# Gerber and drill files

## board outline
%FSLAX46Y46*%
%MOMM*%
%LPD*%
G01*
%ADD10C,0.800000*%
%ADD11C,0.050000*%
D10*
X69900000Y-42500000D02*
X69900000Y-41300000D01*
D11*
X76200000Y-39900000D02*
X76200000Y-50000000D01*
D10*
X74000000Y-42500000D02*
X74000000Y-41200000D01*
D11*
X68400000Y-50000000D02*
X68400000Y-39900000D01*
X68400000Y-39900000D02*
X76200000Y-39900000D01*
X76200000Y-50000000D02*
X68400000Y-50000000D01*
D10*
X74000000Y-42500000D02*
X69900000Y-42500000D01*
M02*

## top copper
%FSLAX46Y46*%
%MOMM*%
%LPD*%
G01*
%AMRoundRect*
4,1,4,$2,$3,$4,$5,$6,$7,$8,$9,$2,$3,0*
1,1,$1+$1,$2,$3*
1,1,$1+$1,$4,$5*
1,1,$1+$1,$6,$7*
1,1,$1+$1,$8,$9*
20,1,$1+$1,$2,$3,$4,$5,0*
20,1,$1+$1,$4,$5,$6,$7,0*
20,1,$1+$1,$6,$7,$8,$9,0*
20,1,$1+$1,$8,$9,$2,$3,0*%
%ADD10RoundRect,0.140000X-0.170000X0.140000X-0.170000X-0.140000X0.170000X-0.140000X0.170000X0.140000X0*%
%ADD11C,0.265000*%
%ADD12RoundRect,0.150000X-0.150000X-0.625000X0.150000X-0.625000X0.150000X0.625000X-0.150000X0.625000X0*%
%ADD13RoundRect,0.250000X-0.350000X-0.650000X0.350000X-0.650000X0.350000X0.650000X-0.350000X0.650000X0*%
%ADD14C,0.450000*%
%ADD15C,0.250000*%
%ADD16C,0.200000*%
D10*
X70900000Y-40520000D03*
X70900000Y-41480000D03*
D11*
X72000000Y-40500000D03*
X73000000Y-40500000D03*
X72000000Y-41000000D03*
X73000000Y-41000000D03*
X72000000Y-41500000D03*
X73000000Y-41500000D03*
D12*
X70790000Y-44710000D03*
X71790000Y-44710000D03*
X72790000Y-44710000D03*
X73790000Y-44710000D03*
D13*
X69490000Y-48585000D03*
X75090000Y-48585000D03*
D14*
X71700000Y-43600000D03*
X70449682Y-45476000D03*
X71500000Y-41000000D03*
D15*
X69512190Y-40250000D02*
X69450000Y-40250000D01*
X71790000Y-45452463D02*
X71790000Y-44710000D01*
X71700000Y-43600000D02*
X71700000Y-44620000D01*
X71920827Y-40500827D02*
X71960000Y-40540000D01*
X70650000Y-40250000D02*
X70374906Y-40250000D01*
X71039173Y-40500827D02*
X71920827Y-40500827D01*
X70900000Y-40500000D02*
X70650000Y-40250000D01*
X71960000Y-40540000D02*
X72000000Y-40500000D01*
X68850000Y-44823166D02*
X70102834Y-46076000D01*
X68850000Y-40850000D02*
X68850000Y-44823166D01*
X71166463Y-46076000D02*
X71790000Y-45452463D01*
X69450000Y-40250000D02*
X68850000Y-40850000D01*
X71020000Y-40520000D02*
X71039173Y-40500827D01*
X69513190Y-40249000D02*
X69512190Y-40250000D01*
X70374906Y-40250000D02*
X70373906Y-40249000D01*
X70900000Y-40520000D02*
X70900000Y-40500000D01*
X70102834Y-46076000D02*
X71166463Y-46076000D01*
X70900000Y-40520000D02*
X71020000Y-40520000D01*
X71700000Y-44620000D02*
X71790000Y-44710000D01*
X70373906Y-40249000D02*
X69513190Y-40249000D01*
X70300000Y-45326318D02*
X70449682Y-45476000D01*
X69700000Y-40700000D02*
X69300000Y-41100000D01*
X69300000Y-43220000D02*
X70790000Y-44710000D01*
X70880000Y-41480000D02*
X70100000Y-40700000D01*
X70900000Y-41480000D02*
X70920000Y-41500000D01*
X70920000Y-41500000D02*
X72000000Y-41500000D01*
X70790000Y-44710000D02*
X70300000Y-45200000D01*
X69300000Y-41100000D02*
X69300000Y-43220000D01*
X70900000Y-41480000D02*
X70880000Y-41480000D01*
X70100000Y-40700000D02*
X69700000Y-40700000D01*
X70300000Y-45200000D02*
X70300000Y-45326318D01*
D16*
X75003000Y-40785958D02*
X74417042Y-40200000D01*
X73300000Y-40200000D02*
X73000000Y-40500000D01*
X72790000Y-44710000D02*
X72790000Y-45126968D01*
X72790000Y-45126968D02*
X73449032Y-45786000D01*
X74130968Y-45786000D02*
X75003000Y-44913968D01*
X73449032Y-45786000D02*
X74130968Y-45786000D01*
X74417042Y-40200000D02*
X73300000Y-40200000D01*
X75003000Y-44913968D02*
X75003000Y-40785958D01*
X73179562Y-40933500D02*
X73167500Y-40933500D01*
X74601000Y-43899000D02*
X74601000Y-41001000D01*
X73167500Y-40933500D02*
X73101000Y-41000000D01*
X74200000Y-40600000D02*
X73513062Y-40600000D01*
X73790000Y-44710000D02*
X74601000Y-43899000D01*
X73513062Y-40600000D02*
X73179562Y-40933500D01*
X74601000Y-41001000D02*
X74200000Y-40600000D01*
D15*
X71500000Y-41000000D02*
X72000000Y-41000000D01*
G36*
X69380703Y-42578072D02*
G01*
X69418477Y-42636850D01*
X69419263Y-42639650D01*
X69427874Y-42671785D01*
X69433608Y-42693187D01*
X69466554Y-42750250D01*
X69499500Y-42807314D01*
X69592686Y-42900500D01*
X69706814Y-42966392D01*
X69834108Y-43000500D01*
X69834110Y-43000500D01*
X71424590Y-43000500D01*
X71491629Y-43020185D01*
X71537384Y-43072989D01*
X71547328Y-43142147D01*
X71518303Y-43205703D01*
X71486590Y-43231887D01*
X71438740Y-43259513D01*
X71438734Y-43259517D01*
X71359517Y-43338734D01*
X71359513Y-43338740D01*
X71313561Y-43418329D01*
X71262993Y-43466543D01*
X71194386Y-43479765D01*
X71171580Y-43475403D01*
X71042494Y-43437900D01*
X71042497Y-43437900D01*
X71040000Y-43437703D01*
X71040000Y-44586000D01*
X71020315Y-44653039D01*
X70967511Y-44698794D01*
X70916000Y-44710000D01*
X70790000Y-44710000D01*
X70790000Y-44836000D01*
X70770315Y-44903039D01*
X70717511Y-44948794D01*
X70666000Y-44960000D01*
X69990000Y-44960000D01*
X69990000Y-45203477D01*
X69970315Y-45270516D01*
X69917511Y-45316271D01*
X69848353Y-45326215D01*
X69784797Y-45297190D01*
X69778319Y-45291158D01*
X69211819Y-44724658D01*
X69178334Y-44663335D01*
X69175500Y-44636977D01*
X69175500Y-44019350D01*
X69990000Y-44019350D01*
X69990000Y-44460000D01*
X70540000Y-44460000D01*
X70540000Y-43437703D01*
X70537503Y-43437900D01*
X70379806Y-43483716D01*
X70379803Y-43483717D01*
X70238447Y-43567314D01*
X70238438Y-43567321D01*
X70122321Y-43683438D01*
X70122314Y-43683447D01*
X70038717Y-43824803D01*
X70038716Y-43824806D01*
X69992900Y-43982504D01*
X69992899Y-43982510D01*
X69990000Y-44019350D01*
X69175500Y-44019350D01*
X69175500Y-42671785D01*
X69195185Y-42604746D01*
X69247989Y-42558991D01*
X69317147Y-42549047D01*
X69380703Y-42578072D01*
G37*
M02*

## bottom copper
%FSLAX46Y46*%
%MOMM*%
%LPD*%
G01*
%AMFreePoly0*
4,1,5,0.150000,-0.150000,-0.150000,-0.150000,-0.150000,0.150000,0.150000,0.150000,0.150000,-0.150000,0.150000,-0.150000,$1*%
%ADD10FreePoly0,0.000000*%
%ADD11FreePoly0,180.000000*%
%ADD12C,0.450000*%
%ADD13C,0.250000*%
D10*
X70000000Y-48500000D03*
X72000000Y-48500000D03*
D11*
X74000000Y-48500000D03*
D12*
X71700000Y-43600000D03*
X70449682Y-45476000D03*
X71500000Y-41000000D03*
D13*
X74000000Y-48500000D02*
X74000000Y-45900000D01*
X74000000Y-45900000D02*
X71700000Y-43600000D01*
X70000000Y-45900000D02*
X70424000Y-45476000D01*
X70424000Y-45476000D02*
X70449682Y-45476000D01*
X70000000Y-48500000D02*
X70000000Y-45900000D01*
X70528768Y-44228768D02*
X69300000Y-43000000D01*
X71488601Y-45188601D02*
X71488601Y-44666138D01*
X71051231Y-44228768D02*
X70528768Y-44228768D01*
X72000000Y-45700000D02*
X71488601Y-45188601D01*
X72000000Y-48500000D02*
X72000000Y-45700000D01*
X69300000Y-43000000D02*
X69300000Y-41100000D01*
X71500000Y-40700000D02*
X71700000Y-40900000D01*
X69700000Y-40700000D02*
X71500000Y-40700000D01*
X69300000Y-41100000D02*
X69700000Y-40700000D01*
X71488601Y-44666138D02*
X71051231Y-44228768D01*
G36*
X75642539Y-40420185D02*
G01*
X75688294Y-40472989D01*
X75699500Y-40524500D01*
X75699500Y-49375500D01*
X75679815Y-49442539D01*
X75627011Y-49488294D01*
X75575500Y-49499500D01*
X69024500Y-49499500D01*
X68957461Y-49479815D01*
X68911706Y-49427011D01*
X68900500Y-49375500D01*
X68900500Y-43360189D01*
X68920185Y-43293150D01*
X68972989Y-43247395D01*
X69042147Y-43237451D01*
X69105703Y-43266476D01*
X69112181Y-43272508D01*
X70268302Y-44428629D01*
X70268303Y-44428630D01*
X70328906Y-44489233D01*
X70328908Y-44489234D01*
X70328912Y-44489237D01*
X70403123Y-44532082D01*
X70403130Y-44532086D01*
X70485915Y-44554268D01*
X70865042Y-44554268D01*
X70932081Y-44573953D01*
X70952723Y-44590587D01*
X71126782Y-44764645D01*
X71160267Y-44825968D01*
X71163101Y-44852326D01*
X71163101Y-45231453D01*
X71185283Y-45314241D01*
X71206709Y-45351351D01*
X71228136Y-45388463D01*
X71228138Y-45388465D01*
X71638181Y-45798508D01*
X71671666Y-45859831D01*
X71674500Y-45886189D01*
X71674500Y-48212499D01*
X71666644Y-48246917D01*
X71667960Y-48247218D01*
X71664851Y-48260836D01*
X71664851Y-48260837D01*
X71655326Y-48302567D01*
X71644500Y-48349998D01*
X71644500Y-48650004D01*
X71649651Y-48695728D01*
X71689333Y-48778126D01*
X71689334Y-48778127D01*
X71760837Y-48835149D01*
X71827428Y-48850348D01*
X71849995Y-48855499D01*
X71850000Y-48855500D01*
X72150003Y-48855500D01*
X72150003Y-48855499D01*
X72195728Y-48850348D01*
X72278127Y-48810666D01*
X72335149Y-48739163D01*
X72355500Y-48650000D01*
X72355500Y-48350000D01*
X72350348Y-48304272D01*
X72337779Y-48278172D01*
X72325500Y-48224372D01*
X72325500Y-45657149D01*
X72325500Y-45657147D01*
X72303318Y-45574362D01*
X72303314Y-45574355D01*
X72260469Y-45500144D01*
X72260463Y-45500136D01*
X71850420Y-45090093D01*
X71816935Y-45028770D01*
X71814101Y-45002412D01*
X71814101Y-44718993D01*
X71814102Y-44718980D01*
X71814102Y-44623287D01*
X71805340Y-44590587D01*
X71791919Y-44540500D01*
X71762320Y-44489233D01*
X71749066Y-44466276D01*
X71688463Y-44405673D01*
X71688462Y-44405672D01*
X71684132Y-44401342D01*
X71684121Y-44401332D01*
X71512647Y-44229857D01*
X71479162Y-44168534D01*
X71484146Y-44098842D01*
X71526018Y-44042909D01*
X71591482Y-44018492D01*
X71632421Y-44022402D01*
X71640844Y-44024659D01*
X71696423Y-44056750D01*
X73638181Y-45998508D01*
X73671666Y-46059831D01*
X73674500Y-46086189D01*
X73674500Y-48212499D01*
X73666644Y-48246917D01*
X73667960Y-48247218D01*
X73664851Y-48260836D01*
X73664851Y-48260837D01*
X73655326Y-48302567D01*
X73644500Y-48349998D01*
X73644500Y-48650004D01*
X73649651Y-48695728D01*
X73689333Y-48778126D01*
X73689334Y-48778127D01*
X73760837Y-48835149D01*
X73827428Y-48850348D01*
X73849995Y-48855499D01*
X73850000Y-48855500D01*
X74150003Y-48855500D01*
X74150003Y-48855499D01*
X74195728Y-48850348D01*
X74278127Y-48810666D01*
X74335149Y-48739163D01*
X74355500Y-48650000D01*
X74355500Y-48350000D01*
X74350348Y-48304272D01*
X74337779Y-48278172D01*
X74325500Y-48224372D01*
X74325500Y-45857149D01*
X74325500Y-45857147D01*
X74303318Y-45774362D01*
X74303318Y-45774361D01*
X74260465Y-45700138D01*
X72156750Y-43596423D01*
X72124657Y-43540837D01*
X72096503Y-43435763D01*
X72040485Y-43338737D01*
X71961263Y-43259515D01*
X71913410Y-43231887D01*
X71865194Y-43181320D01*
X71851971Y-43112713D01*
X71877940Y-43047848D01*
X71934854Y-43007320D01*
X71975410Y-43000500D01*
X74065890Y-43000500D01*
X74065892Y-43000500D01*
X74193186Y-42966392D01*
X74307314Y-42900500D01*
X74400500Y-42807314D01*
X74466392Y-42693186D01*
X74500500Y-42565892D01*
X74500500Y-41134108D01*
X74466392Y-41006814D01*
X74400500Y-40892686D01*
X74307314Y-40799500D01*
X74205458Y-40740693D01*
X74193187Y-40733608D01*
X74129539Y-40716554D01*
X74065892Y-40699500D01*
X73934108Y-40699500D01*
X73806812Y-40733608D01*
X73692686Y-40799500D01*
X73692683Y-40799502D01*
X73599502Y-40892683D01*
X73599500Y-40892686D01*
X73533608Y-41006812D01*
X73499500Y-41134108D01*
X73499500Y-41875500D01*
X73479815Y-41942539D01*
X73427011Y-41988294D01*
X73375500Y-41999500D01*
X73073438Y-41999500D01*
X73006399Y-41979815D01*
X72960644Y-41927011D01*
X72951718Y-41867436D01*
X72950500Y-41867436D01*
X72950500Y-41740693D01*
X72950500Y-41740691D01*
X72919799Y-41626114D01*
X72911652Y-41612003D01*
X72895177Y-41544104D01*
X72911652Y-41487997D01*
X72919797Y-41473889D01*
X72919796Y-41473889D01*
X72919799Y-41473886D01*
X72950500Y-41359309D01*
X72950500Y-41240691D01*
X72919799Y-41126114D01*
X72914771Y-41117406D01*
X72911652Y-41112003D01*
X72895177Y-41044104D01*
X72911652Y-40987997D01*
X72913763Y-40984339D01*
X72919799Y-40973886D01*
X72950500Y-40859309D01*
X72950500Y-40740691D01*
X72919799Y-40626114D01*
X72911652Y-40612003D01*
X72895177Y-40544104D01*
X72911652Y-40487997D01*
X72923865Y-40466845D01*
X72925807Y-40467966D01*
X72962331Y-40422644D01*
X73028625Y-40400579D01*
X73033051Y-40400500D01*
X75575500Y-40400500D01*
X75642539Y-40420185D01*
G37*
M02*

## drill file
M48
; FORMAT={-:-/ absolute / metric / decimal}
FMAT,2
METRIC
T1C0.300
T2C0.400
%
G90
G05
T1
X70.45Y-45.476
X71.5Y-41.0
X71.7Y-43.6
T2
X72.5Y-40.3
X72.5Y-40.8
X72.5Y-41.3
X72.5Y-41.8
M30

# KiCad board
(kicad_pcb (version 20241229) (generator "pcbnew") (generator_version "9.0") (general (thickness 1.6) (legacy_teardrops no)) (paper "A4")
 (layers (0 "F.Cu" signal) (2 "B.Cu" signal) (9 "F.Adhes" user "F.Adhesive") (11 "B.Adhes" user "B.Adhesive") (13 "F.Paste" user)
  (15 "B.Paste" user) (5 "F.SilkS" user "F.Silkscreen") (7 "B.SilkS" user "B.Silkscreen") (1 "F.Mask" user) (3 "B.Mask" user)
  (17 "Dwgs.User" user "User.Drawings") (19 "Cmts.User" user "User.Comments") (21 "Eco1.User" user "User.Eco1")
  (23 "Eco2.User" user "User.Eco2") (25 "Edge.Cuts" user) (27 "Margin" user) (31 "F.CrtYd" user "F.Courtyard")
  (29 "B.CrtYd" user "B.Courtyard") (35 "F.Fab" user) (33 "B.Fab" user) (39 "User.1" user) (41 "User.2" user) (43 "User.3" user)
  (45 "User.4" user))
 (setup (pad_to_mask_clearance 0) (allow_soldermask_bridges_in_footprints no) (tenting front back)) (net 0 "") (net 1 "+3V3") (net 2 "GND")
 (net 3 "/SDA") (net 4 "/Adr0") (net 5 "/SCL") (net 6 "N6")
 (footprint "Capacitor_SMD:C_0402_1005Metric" (layer "F.Cu") (at 70.9 41 -90)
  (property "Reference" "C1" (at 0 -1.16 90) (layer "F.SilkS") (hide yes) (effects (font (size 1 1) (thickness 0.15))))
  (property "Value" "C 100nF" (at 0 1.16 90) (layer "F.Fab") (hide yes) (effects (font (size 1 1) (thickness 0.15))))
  (pad "1" smd roundrect (at -0.48 0 270) (size 0.56 0.62) (layers "F.Cu" "F.Mask" "F.Paste") (roundrect_rratio 0.25) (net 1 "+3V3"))
  (pad "2" smd roundrect (at 0.48 0 270) (size 0.56 0.62) (layers "F.Cu" "F.Mask" "F.Paste") (roundrect_rratio 0.25) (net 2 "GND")))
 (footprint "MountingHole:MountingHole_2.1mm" (layer "F.Cu") (at 72.5 40.3)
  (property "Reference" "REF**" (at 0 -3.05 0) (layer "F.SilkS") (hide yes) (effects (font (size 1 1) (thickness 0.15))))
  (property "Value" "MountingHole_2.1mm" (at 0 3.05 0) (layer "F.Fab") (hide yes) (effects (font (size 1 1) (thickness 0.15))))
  (pad "" np_thru_hole circle (at 0 0) (size 0.4 0.4) (drill 0.4) (layers "*.Mask")))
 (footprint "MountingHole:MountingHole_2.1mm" (layer "F.Cu") (at 72.5 41.3)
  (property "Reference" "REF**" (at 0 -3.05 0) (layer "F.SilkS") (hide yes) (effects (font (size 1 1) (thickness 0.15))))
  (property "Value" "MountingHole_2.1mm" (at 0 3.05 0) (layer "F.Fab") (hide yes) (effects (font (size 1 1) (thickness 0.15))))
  (pad "" np_thru_hole circle (at 0 0) (size 0.4 0.4) (drill 0.4) (layers "*.Cu" "*.Mask")))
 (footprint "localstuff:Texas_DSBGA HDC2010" (layer "F.Cu") (at 72.5 41)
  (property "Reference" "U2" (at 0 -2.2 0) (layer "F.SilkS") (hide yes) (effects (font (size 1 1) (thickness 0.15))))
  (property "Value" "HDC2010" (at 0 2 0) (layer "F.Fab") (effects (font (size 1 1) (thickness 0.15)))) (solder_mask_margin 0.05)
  (pad "" smd rect (at -0.5 -0.5) (size 0.3 0.3) (layers "F.Paste"))
  (pad "" smd rect (at -0.5 0) (size 0.3 0.3) (layers "F.Paste"))
  (pad "" smd rect (at -0.5 0.5) (size 0.3 0.3) (layers "F.Paste"))
  (pad "" smd rect (at 0.5 -0.5) (size 0.3 0.3) (layers "F.Paste"))
  (pad "" smd rect (at 0.5 0) (size 0.3 0.3) (layers "F.Paste"))
  (pad "" smd rect (at 0.5 0.5) (size 0.3 0.3) (layers "F.Paste"))
  (pad "A1" smd circle (at -0.5 -0.5) (size 0.265 0.265) (layers "F.Cu" "F.Mask") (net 1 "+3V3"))
  (pad "A2" smd circle (at 0.5 -0.5) (size 0.265 0.265) (layers "F.Cu" "F.Mask") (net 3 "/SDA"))
  (pad "B1" smd circle (at -0.5 0) (size 0.265 0.265) (layers "F.Cu" "F.Mask") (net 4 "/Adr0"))
  (pad "B2" smd circle (at 0.5 0) (size 0.265 0.265) (layers "F.Cu" "F.Mask") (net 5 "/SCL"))
  (pad "C1" smd circle (at -0.5 0.5) (size 0.265 0.265) (layers "F.Cu" "F.Mask") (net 2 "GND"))
  (pad "C2" smd circle (at 0.5 0.5) (size 0.265 0.265) (layers "F.Cu" "F.Mask") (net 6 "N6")))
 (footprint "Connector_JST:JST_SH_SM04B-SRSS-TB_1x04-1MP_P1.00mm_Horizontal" (layer "F.Cu") (at 72.29 46.71)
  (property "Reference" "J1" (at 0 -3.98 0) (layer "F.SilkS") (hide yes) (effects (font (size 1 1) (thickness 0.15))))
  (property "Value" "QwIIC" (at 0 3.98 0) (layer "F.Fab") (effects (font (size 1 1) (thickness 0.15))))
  (pad "1" smd roundrect (at -1.5 -2) (size 0.6 1.55) (layers "F.Cu" "F.Mask" "F.Paste") (roundrect_rratio 0.25) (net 2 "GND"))
  (pad "2" smd roundrect (at -0.5 -2) (size 0.6 1.55) (layers "F.Cu" "F.Mask" "F.Paste") (roundrect_rratio 0.25) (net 1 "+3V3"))
  (pad "3" smd roundrect (at 0.5 -2) (size 0.6 1.55) (layers "F.Cu" "F.Mask" "F.Paste") (roundrect_rratio 0.25) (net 3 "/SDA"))
  (pad "4" smd roundrect (at 1.5 -2) (size 0.6 1.55) (layers "F.Cu" "F.Mask" "F.Paste") (roundrect_rratio 0.25) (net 5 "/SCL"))
  (pad "MP" smd roundrect (at -2.8 1.875) (size 1.2 1.8) (layers "F.Cu" "F.Mask" "F.Paste") (roundrect_rratio 0.208333))
  (pad "MP" smd roundrect (at 2.8 1.875) (size 1.2 1.8) (layers "F.Cu" "F.Mask" "F.Paste") (roundrect_rratio 0.208333)))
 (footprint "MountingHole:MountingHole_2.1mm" (layer "F.Cu") (at 72.5 40.8)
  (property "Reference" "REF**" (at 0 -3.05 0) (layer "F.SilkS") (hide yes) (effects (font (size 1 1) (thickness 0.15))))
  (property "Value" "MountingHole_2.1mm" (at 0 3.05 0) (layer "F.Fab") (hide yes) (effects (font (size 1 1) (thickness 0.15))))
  (pad "" np_thru_hole circle (at 0 0) (size 0.4 0.4) (drill 0.4) (layers "*.Cu" "*.Mask")))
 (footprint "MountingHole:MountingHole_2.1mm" (layer "F.Cu") (at 72.5 41.8)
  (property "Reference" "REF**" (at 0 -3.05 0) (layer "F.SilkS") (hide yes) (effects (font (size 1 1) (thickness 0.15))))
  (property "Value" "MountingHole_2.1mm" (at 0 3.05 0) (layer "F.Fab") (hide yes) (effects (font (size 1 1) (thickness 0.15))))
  (pad "" np_thru_hole circle (at 0 0) (size 0.4 0.4) (drill 0.4) (layers "*.Cu" "*.Mask")))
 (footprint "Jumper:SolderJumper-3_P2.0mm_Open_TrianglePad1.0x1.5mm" (layer "B.Cu") (at 72 48.5)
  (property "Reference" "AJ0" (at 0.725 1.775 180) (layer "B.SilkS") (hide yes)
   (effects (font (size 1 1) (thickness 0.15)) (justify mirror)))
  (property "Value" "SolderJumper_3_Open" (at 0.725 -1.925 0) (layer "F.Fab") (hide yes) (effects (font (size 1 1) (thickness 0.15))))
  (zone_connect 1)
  (pad "1" smd custom (at -2 0) (size 0.3 0.3) (layers "B.Cu" "B.Mask") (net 2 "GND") (zone_connect 2) (thermal_bridge_angle 45)
   (options (clearance outline) (anchor rect)) (primitives))
  (pad "2" smd custom (at 0 0) (size 0.3 0.3) (layers "B.Cu") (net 4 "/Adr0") (zone_connect 2) (thermal_bridge_angle 45)
   (options (clearance outline) (anchor rect)) (primitives))
  (pad "3" smd custom (at 2 0 180) (size 0.3 0.3) (layers "B.Cu" "B.Mask") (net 1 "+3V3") (zone_connect 2) (thermal_bridge_angle 45)
   (options (clearance outline) (anchor rect)) (primitives)))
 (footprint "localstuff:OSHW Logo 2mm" (layer "B.Cu") (at 75.003 44.913968 180)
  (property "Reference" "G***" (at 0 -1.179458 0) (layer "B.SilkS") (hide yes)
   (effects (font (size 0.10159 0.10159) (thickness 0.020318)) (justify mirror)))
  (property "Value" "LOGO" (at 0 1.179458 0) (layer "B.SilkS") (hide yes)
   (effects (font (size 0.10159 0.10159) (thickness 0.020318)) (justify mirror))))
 (gr_line (start 69.9 42.5) (end 69.9 41.3) (stroke (width 0.8) (type solid)) (layer "Edge.Cuts"))
 (gr_line (start 76.2 39.9) (end 76.2 50) (stroke (width 0.05) (type default)) (layer "Edge.Cuts"))
 (gr_line (start 74 42.5) (end 74 41.2) (stroke (width 0.8) (type solid)) (layer "Edge.Cuts"))
 (gr_line (start 68.4 50) (end 68.4 39.9) (stroke (width 0.05) (type default)) (layer "Edge.Cuts"))
 (gr_line (start 68.4 39.9) (end 76.2 39.9) (stroke (width 0.05) (type default)) (layer "Edge.Cuts"))
 (gr_line (start 76.2 50) (end 68.4 50) (stroke (width 0.05) (type default)) (layer "Edge.Cuts"))
 (gr_line (start 74 42.5) (end 69.9 42.5) (stroke (width 0.8) (type solid)) (layer "Edge.Cuts"))
 (segment (start 69.51219 40.25) (end 69.45 40.25) (width 0.25) (layer "F.Cu") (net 1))
 (segment (start 71.79 45.452463) (end 71.79 44.71) (width 0.25) (layer "F.Cu") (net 1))
 (segment (start 71.7 43.6) (end 71.7 44.62) (width 0.25) (layer "F.Cu") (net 1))
 (segment (start 71.920827 40.500827) (end 71.96 40.54) (width 0.25) (layer "F.Cu") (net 1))
 (segment (start 70.65 40.25) (end 70.374906 40.25) (width 0.25) (layer "F.Cu") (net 1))
 (segment (start 71.039173 40.500827) (end 71.920827 40.500827) (width 0.25) (layer "F.Cu") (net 1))
 (segment (start 70.9 40.5) (end 70.65 40.25) (width 0.25) (layer "F.Cu") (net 1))
 (segment (start 71.96 40.54) (end 72 40.5) (width 0.25) (layer "F.Cu") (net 1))
 (segment (start 68.85 44.823166) (end 70.102834 46.076) (width 0.25) (layer "F.Cu") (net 1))
 (segment (start 68.85 40.85) (end 68.85 44.823166) (width 0.25) (layer "F.Cu") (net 1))
 (segment (start 71.166463 46.076) (end 71.79 45.452463) (width 0.25) (layer "F.Cu") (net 1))
 (segment (start 69.45 40.25) (end 68.85 40.85) (width 0.25) (layer "F.Cu") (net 1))
 (segment (start 71.02 40.52) (end 71.039173 40.500827) (width 0.25) (layer "F.Cu") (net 1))
 (segment (start 69.51319 40.249) (end 69.51219 40.25) (width 0.25) (layer "F.Cu") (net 1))
 (segment (start 70.374906 40.25) (end 70.373906 40.249) (width 0.25) (layer "F.Cu") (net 1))
 (segment (start 70.9 40.52) (end 70.9 40.5) (width 0.25) (layer "F.Cu") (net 1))
 (segment (start 70.102834 46.076) (end 71.166463 46.076) (width 0.25) (layer "F.Cu") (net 1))
 (segment (start 70.9 40.52) (end 71.02 40.52) (width 0.25) (layer "F.Cu") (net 1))
 (segment (start 71.7 44.62) (end 71.79 44.71) (width 0.25) (layer "F.Cu") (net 1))
 (segment (start 70.373906 40.249) (end 69.51319 40.249) (width 0.25) (layer "F.Cu") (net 1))
 (via (at 71.7 43.6) (size 0.45) (drill 0.3) (layers "F.Cu" "B.Cu") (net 1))
 (segment (start 74 48.5) (end 74 45.9) (width 0.25) (layer "B.Cu") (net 1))
 (segment (start 74 45.9) (end 71.7 43.6) (width 0.25) (layer "B.Cu") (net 1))
 (segment (start 70.3 45.326318) (end 70.449682 45.476) (width 0.25) (layer "F.Cu") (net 2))
 (segment (start 69.7 40.7) (end 69.3 41.1) (width 0.25) (layer "F.Cu") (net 2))
 (segment (start 69.3 43.22) (end 70.79 44.71) (width 0.25) (layer "F.Cu") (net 2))
 (segment (start 70.88 41.48) (end 70.1 40.7) (width 0.25) (layer "F.Cu") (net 2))
 (segment (start 70.9 41.48) (end 70.92 41.5) (width 0.25) (layer "F.Cu") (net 2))
 (segment (start 70.92 41.5) (end 72 41.5) (width 0.25) (layer "F.Cu") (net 2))
 (segment (start 70.79 44.71) (end 70.3 45.2) (width 0.25) (layer "F.Cu") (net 2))
 (segment (start 69.3 41.1) (end 69.3 43.22) (width 0.25) (layer "F.Cu") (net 2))
 (segment (start 70.9 41.48) (end 70.88 41.48) (width 0.25) (layer "F.Cu") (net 2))
 (segment (start 70.1 40.7) (end 69.7 40.7) (width 0.25) (layer "F.Cu") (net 2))
 (segment (start 70.3 45.2) (end 70.3 45.326318) (width 0.25) (layer "F.Cu") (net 2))
 (via (at 70.449682 45.476) (size 0.45) (drill 0.3) (layers "F.Cu" "B.Cu") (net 2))
 (segment (start 70 45.9) (end 70.424 45.476) (width 0.25) (layer "B.Cu") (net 2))
 (segment (start 70.424 45.476) (end 70.449682 45.476) (width 0.25) (layer "B.Cu") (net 2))
 (segment (start 70 48.5) (end 70 45.9) (width 0.25) (layer "B.Cu") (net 2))
 (segment (start 75.003 40.785958) (end 74.417042 40.2) (width 0.2) (layer "F.Cu") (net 3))
 (segment (start 73.3 40.2) (end 73 40.5) (width 0.2) (layer "F.Cu") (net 3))
 (segment (start 72.79 44.71) (end 72.79 45.126968) (width 0.2) (layer "F.Cu") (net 3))
 (segment (start 72.79 45.126968) (end 73.449032 45.786) (width 0.2) (layer "F.Cu") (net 3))
 (segment (start 74.130968 45.786) (end 75.003 44.913968) (width 0.2) (layer "F.Cu") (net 3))
 (segment (start 73.449032 45.786) (end 74.130968 45.786) (width 0.2) (layer "F.Cu") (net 3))
 (segment (start 74.417042 40.2) (end 73.3 40.2) (width 0.2) (layer "F.Cu") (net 3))
 (segment (start 75.003 44.913968) (end 75.003 40.785958) (width 0.2) (layer "F.Cu") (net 3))
 (segment (start 73.179562 40.9335) (end 73.1675 40.9335) (width 0.2) (layer "F.Cu") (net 5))
 (segment (start 74.601 43.899) (end 74.601 41.001) (width 0.2) (layer "F.Cu") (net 5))
 (segment (start 73.1675 40.9335) (end 73.101 41) (width 0.2) (layer "F.Cu") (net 5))
 (segment (start 74.2 40.6) (end 73.513062 40.6) (width 0.2) (layer "F.Cu") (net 5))
 (segment (start 73.79 44.71) (end 74.601 43.899) (width 0.2) (layer "F.Cu") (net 5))
 (segment (start 73.513062 40.6) (end 73.179562 40.9335) (width 0.2) (layer "F.Cu") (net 5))
 (segment (start 74.601 41.001) (end 74.2 40.6) (width 0.2) (layer "F.Cu") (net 5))
 (segment (start 71.5 41) (end 72 41) (width 0.25) (layer "F.Cu") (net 4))
 (via (at 71.5 41) (size 0.45) (drill 0.3) (layers "F.Cu" "B.Cu") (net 4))
 (segment (start 70.528768 44.228768) (end 69.3 43) (width 0.25) (layer "B.Cu") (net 4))
 (segment (start 71.488601 45.188601) (end 71.488601 44.666138) (width 0.25) (layer "B.Cu") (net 4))
 (segment (start 71.051231 44.228768) (end 70.528768 44.228768) (width 0.25) (layer "B.Cu") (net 4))
 (segment (start 72 45.7) (end 71.488601 45.188601) (width 0.25) (layer "B.Cu") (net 4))
 (segment (start 72 48.5) (end 72 45.7) (width 0.25) (layer "B.Cu") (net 4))
 (segment (start 69.3 43) (end 69.3 41.1) (width 0.25) (layer "B.Cu") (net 4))
 (segment (start 71.5 40.7) (end 71.7 40.9) (width 0.25) (layer "B.Cu") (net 4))
 (segment (start 69.7 40.7) (end 71.5 40.7) (width 0.25) (layer "B.Cu") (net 4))
 (segment (start 69.3 41.1) (end 69.7 40.7) (width 0.25) (layer "B.Cu") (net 4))
 (segment (start 71.488601 44.666138) (end 71.051231 44.228768) (width 0.25) (layer "B.Cu") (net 4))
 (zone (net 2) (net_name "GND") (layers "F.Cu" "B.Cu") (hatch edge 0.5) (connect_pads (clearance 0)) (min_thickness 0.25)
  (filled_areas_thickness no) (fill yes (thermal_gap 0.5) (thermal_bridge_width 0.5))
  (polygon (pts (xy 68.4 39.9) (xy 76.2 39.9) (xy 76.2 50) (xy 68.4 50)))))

